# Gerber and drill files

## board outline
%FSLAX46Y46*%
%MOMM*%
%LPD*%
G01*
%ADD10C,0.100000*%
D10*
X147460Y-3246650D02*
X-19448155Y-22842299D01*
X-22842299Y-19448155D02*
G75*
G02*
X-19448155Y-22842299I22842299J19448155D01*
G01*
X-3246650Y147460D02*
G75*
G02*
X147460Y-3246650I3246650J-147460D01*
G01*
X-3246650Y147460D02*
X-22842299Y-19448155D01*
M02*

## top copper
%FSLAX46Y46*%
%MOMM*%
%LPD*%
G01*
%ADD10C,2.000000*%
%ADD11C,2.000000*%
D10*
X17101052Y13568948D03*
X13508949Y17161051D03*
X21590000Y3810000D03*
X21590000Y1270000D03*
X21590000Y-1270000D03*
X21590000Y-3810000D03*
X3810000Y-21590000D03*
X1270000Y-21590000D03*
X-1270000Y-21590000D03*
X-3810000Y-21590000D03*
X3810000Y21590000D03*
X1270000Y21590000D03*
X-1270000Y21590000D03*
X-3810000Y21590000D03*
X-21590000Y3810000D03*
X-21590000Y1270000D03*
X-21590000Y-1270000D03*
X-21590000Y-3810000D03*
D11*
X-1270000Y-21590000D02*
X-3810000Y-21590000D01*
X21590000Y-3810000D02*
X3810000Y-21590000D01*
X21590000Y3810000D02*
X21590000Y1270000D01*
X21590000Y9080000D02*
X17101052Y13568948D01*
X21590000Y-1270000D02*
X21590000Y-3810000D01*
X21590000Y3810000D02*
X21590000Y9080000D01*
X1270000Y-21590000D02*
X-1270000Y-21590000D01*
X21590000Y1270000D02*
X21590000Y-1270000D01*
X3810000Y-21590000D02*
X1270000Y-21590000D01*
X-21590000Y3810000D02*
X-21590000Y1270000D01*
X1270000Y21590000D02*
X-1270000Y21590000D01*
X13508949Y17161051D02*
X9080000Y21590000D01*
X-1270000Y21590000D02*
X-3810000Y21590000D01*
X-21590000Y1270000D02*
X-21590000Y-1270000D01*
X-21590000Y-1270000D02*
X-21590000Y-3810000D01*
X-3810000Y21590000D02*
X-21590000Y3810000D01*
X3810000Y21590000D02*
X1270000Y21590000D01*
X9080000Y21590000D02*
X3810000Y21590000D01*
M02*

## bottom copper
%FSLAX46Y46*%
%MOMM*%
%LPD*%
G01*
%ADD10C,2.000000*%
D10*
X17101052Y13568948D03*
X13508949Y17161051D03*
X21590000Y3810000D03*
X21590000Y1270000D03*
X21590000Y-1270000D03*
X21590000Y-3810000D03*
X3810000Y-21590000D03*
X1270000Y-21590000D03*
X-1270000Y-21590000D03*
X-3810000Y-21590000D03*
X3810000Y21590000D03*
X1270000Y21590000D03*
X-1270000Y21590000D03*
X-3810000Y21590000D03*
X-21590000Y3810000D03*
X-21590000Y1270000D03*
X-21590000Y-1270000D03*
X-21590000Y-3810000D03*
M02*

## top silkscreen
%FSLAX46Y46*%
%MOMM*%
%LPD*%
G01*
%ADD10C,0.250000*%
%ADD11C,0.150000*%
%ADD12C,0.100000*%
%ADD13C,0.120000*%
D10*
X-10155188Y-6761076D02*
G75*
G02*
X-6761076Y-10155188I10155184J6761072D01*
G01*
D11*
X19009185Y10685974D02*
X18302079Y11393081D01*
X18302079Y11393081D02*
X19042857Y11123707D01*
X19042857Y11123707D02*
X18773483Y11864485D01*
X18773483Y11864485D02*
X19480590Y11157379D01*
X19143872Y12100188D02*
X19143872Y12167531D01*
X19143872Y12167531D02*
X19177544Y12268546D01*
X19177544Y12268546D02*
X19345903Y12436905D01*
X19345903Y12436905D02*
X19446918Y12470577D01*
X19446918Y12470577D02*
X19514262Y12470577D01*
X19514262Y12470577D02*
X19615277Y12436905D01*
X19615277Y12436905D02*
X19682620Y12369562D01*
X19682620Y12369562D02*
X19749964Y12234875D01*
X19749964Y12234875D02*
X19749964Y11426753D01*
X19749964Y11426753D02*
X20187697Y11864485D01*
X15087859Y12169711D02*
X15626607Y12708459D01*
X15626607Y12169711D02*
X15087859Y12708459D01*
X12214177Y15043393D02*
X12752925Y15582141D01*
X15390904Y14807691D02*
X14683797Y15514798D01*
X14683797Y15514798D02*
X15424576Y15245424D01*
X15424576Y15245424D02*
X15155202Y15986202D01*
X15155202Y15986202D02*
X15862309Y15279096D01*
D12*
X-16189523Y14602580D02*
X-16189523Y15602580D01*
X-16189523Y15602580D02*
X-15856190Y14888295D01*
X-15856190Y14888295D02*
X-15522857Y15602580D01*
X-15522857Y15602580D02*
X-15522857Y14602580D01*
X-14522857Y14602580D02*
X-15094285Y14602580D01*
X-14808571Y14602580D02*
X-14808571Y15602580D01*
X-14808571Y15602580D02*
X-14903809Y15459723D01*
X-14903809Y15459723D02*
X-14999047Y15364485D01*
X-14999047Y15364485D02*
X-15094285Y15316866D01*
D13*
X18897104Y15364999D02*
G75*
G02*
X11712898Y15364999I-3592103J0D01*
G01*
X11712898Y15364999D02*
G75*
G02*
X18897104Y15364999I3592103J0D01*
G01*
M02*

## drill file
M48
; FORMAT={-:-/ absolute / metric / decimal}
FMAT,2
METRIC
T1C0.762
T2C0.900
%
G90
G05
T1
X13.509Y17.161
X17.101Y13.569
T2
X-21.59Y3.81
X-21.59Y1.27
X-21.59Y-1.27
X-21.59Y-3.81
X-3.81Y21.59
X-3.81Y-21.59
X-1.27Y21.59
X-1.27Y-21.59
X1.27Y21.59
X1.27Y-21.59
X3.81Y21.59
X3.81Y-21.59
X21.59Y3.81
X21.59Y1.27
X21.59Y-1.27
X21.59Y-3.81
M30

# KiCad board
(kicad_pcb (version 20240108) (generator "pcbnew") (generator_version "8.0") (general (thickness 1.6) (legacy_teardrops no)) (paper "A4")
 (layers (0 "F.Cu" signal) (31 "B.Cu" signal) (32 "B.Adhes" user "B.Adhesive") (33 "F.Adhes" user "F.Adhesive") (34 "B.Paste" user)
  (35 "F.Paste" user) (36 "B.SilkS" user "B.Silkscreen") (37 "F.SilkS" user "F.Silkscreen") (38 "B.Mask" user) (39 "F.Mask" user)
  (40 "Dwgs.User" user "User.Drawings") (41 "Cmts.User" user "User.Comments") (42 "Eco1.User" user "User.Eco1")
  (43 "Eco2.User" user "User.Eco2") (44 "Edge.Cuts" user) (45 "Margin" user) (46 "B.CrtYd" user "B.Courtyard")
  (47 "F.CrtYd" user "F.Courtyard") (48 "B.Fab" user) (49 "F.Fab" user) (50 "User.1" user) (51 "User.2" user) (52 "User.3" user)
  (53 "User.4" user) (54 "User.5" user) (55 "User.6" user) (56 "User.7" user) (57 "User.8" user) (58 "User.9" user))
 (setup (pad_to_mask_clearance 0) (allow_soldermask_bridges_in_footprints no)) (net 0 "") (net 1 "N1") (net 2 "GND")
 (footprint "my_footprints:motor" (layer "F.Cu") (at 18.897103 -11.772897 -135)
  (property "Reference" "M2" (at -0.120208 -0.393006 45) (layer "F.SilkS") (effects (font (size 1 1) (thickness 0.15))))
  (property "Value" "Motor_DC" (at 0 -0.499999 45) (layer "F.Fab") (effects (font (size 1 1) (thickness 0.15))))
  (fp_circle (center 0 5.079999) (end 2.54 7.62) (stroke (width 0.12) (type solid)) (fill none) (layer "F.SilkS"))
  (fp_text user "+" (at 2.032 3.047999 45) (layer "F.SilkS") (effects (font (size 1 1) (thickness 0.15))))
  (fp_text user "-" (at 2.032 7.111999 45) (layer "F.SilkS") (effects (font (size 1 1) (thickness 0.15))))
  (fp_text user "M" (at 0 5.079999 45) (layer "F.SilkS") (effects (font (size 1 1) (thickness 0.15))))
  (pad "1" thru_hole circle (at 0 2.54 225) (size 2 2) (drill 0.762) (layers "*.Cu" "*.Mask") (remove_unused_layers no) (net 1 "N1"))
  (pad "2" thru_hole circle (at 0 7.62 225) (size 2 2) (drill 0.762) (layers "*.Cu" "*.Mask") (remove_unused_layers no) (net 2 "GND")))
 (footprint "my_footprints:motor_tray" (layer "F.Cu") (at 0 0 -90)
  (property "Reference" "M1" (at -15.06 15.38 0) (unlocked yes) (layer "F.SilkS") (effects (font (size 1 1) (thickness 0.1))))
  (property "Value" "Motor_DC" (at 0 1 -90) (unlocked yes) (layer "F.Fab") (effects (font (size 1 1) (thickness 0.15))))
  (pad "1" thru_hole circle (at -3.81 -21.59 270) (size 2 2) (drill 0.9) (layers "*.Cu" "*.Mask") (remove_unused_layers no) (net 1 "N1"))
  (pad "1" thru_hole circle (at -1.27 -21.59 270) (size 2 2) (drill 0.9) (layers "*.Cu" "*.Mask") (remove_unused_layers no) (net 1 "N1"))
  (pad "1" thru_hole circle (at 1.27 -21.59 270) (size 2 2) (drill 0.9) (layers "*.Cu" "*.Mask") (remove_unused_layers no) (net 1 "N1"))
  (pad "1" thru_hole circle (at 3.81 -21.59 270) (size 2 2) (drill 0.9) (layers "*.Cu" "*.Mask") (remove_unused_layers no) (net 1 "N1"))
  (pad "1" thru_hole circle (at 21.59 -3.81 270) (size 2 2) (drill 0.9) (layers "*.Cu" "*.Mask") (remove_unused_layers no) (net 1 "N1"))
  (pad "1" thru_hole circle (at 21.59 -1.27 270) (size 2 2) (drill 0.9) (layers "*.Cu" "*.Mask") (remove_unused_layers no) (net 1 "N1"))
  (pad "1" thru_hole circle (at 21.59 1.27 270) (size 2 2) (drill 0.9) (layers "*.Cu" "*.Mask") (remove_unused_layers no) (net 1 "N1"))
  (pad "1" thru_hole circle (at 21.59 3.81 270) (size 2 2) (drill 0.9) (layers "*.Cu" "*.Mask") (remove_unused_layers no) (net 1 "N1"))
  (pad "2" thru_hole circle (at -21.59 -3.81 270) (size 2 2) (drill 0.9) (layers "*.Cu" "*.Mask") (remove_unused_layers no) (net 2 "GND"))
  (pad "2" thru_hole circle (at -21.59 -1.27 270) (size 2 2) (drill 0.9) (layers "*.Cu" "*.Mask") (remove_unused_layers no) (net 2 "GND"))
  (pad "2" thru_hole circle (at -21.59 1.27 270) (size 2 2) (drill 0.9) (layers "*.Cu" "*.Mask") (remove_unused_layers no) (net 2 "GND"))
  (pad "2" thru_hole circle (at -21.59 3.81 270) (size 2 2) (drill 0.9) (layers "*.Cu" "*.Mask") (remove_unused_layers no) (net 2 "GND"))
  (pad "2" thru_hole circle (at -3.81 21.59 270) (size 2 2) (drill 0.9) (layers "*.Cu" "*.Mask") (remove_unused_layers no) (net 2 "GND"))
  (pad "2" thru_hole circle (at -1.27 21.59 270) (size 2 2) (drill 0.9) (layers "*.Cu" "*.Mask") (remove_unused_layers no) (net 2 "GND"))
  (pad "2" thru_hole circle (at 1.27 21.59 270) (size 2 2) (drill 0.9) (layers "*.Cu" "*.Mask") (remove_unused_layers no) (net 2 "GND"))
  (pad "2" thru_hole circle (at 3.81 21.59 270) (size 2 2) (drill 0.9) (layers "*.Cu" "*.Mask") (remove_unused_layers no) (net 2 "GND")))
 (gr_arc (start -10.155188 6.761076) (mid 8.626695 -8.626695) (end -6.761076 10.155188) (stroke (width 0.25) (type default))
  (layer "F.SilkS"))
 (gr_line (start 0.14746 3.24665) (end -19.448155 22.842299) (stroke (width 0.1) (type default)) (layer "Edge.Cuts"))
 (gr_arc (start -22.842299 19.448155) (mid 21.213219 -21.213219) (end -19.448155 22.842299) (stroke (width 0.1) (type default))
  (layer "Edge.Cuts"))
 (gr_arc (start -3.24665 -0.14746) (mid 2.298095 -2.298095) (end 0.14746 3.24665) (stroke (width 0.1) (type default)) (layer "Edge.Cuts"))
 (gr_line (start -3.24665 -0.14746) (end -22.842299 19.448155) (stroke (width 0.1) (type default)) (layer "Edge.Cuts"))
 (segment (start -1.27 21.59) (end -3.81 21.59) (width 2) (layer "F.Cu") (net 1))
 (segment (start 21.59 3.81) (end 3.81 21.59) (width 2) (layer "F.Cu") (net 1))
 (segment (start 21.59 -3.81) (end 21.59 -1.27) (width 2) (layer "F.Cu") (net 1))
 (segment (start 21.59 -9.08) (end 17.101052 -13.568948) (width 2) (layer "F.Cu") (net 1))
 (segment (start 21.59 1.27) (end 21.59 3.81) (width 2) (layer "F.Cu") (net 1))
 (segment (start 21.59 -3.81) (end 21.59 -9.08) (width 2) (layer "F.Cu") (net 1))
 (segment (start 1.27 21.59) (end -1.27 21.59) (width 2) (layer "F.Cu") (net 1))
 (segment (start 21.59 -1.27) (end 21.59 1.27) (width 2) (layer "F.Cu") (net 1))
 (segment (start 3.81 21.59) (end 1.27 21.59) (width 2) (layer "F.Cu") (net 1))
 (segment (start -21.59 -3.81) (end -21.59 -1.27) (width 2) (layer "F.Cu") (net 2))
 (segment (start 1.27 -21.59) (end -1.27 -21.59) (width 2) (layer "F.Cu") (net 2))
 (segment (start 13.508949 -17.161051) (end 9.08 -21.59) (width 2) (layer "F.Cu") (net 2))
 (segment (start -1.27 -21.59) (end -3.81 -21.59) (width 2) (layer "F.Cu") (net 2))
 (segment (start -21.59 -1.27) (end -21.59 1.27) (width 2) (layer "F.Cu") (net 2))
 (segment (start -21.59 1.27) (end -21.59 3.81) (width 2) (layer "F.Cu") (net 2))
 (segment (start -3.81 -21.59) (end -21.59 -3.81) (width 2) (layer "F.Cu") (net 2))
 (segment (start 3.81 -21.59) (end 1.27 -21.59) (width 2) (layer "F.Cu") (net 2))
 (segment (start 9.08 -21.59) (end 3.81 -21.59) (width 2) (layer "F.Cu") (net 2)))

